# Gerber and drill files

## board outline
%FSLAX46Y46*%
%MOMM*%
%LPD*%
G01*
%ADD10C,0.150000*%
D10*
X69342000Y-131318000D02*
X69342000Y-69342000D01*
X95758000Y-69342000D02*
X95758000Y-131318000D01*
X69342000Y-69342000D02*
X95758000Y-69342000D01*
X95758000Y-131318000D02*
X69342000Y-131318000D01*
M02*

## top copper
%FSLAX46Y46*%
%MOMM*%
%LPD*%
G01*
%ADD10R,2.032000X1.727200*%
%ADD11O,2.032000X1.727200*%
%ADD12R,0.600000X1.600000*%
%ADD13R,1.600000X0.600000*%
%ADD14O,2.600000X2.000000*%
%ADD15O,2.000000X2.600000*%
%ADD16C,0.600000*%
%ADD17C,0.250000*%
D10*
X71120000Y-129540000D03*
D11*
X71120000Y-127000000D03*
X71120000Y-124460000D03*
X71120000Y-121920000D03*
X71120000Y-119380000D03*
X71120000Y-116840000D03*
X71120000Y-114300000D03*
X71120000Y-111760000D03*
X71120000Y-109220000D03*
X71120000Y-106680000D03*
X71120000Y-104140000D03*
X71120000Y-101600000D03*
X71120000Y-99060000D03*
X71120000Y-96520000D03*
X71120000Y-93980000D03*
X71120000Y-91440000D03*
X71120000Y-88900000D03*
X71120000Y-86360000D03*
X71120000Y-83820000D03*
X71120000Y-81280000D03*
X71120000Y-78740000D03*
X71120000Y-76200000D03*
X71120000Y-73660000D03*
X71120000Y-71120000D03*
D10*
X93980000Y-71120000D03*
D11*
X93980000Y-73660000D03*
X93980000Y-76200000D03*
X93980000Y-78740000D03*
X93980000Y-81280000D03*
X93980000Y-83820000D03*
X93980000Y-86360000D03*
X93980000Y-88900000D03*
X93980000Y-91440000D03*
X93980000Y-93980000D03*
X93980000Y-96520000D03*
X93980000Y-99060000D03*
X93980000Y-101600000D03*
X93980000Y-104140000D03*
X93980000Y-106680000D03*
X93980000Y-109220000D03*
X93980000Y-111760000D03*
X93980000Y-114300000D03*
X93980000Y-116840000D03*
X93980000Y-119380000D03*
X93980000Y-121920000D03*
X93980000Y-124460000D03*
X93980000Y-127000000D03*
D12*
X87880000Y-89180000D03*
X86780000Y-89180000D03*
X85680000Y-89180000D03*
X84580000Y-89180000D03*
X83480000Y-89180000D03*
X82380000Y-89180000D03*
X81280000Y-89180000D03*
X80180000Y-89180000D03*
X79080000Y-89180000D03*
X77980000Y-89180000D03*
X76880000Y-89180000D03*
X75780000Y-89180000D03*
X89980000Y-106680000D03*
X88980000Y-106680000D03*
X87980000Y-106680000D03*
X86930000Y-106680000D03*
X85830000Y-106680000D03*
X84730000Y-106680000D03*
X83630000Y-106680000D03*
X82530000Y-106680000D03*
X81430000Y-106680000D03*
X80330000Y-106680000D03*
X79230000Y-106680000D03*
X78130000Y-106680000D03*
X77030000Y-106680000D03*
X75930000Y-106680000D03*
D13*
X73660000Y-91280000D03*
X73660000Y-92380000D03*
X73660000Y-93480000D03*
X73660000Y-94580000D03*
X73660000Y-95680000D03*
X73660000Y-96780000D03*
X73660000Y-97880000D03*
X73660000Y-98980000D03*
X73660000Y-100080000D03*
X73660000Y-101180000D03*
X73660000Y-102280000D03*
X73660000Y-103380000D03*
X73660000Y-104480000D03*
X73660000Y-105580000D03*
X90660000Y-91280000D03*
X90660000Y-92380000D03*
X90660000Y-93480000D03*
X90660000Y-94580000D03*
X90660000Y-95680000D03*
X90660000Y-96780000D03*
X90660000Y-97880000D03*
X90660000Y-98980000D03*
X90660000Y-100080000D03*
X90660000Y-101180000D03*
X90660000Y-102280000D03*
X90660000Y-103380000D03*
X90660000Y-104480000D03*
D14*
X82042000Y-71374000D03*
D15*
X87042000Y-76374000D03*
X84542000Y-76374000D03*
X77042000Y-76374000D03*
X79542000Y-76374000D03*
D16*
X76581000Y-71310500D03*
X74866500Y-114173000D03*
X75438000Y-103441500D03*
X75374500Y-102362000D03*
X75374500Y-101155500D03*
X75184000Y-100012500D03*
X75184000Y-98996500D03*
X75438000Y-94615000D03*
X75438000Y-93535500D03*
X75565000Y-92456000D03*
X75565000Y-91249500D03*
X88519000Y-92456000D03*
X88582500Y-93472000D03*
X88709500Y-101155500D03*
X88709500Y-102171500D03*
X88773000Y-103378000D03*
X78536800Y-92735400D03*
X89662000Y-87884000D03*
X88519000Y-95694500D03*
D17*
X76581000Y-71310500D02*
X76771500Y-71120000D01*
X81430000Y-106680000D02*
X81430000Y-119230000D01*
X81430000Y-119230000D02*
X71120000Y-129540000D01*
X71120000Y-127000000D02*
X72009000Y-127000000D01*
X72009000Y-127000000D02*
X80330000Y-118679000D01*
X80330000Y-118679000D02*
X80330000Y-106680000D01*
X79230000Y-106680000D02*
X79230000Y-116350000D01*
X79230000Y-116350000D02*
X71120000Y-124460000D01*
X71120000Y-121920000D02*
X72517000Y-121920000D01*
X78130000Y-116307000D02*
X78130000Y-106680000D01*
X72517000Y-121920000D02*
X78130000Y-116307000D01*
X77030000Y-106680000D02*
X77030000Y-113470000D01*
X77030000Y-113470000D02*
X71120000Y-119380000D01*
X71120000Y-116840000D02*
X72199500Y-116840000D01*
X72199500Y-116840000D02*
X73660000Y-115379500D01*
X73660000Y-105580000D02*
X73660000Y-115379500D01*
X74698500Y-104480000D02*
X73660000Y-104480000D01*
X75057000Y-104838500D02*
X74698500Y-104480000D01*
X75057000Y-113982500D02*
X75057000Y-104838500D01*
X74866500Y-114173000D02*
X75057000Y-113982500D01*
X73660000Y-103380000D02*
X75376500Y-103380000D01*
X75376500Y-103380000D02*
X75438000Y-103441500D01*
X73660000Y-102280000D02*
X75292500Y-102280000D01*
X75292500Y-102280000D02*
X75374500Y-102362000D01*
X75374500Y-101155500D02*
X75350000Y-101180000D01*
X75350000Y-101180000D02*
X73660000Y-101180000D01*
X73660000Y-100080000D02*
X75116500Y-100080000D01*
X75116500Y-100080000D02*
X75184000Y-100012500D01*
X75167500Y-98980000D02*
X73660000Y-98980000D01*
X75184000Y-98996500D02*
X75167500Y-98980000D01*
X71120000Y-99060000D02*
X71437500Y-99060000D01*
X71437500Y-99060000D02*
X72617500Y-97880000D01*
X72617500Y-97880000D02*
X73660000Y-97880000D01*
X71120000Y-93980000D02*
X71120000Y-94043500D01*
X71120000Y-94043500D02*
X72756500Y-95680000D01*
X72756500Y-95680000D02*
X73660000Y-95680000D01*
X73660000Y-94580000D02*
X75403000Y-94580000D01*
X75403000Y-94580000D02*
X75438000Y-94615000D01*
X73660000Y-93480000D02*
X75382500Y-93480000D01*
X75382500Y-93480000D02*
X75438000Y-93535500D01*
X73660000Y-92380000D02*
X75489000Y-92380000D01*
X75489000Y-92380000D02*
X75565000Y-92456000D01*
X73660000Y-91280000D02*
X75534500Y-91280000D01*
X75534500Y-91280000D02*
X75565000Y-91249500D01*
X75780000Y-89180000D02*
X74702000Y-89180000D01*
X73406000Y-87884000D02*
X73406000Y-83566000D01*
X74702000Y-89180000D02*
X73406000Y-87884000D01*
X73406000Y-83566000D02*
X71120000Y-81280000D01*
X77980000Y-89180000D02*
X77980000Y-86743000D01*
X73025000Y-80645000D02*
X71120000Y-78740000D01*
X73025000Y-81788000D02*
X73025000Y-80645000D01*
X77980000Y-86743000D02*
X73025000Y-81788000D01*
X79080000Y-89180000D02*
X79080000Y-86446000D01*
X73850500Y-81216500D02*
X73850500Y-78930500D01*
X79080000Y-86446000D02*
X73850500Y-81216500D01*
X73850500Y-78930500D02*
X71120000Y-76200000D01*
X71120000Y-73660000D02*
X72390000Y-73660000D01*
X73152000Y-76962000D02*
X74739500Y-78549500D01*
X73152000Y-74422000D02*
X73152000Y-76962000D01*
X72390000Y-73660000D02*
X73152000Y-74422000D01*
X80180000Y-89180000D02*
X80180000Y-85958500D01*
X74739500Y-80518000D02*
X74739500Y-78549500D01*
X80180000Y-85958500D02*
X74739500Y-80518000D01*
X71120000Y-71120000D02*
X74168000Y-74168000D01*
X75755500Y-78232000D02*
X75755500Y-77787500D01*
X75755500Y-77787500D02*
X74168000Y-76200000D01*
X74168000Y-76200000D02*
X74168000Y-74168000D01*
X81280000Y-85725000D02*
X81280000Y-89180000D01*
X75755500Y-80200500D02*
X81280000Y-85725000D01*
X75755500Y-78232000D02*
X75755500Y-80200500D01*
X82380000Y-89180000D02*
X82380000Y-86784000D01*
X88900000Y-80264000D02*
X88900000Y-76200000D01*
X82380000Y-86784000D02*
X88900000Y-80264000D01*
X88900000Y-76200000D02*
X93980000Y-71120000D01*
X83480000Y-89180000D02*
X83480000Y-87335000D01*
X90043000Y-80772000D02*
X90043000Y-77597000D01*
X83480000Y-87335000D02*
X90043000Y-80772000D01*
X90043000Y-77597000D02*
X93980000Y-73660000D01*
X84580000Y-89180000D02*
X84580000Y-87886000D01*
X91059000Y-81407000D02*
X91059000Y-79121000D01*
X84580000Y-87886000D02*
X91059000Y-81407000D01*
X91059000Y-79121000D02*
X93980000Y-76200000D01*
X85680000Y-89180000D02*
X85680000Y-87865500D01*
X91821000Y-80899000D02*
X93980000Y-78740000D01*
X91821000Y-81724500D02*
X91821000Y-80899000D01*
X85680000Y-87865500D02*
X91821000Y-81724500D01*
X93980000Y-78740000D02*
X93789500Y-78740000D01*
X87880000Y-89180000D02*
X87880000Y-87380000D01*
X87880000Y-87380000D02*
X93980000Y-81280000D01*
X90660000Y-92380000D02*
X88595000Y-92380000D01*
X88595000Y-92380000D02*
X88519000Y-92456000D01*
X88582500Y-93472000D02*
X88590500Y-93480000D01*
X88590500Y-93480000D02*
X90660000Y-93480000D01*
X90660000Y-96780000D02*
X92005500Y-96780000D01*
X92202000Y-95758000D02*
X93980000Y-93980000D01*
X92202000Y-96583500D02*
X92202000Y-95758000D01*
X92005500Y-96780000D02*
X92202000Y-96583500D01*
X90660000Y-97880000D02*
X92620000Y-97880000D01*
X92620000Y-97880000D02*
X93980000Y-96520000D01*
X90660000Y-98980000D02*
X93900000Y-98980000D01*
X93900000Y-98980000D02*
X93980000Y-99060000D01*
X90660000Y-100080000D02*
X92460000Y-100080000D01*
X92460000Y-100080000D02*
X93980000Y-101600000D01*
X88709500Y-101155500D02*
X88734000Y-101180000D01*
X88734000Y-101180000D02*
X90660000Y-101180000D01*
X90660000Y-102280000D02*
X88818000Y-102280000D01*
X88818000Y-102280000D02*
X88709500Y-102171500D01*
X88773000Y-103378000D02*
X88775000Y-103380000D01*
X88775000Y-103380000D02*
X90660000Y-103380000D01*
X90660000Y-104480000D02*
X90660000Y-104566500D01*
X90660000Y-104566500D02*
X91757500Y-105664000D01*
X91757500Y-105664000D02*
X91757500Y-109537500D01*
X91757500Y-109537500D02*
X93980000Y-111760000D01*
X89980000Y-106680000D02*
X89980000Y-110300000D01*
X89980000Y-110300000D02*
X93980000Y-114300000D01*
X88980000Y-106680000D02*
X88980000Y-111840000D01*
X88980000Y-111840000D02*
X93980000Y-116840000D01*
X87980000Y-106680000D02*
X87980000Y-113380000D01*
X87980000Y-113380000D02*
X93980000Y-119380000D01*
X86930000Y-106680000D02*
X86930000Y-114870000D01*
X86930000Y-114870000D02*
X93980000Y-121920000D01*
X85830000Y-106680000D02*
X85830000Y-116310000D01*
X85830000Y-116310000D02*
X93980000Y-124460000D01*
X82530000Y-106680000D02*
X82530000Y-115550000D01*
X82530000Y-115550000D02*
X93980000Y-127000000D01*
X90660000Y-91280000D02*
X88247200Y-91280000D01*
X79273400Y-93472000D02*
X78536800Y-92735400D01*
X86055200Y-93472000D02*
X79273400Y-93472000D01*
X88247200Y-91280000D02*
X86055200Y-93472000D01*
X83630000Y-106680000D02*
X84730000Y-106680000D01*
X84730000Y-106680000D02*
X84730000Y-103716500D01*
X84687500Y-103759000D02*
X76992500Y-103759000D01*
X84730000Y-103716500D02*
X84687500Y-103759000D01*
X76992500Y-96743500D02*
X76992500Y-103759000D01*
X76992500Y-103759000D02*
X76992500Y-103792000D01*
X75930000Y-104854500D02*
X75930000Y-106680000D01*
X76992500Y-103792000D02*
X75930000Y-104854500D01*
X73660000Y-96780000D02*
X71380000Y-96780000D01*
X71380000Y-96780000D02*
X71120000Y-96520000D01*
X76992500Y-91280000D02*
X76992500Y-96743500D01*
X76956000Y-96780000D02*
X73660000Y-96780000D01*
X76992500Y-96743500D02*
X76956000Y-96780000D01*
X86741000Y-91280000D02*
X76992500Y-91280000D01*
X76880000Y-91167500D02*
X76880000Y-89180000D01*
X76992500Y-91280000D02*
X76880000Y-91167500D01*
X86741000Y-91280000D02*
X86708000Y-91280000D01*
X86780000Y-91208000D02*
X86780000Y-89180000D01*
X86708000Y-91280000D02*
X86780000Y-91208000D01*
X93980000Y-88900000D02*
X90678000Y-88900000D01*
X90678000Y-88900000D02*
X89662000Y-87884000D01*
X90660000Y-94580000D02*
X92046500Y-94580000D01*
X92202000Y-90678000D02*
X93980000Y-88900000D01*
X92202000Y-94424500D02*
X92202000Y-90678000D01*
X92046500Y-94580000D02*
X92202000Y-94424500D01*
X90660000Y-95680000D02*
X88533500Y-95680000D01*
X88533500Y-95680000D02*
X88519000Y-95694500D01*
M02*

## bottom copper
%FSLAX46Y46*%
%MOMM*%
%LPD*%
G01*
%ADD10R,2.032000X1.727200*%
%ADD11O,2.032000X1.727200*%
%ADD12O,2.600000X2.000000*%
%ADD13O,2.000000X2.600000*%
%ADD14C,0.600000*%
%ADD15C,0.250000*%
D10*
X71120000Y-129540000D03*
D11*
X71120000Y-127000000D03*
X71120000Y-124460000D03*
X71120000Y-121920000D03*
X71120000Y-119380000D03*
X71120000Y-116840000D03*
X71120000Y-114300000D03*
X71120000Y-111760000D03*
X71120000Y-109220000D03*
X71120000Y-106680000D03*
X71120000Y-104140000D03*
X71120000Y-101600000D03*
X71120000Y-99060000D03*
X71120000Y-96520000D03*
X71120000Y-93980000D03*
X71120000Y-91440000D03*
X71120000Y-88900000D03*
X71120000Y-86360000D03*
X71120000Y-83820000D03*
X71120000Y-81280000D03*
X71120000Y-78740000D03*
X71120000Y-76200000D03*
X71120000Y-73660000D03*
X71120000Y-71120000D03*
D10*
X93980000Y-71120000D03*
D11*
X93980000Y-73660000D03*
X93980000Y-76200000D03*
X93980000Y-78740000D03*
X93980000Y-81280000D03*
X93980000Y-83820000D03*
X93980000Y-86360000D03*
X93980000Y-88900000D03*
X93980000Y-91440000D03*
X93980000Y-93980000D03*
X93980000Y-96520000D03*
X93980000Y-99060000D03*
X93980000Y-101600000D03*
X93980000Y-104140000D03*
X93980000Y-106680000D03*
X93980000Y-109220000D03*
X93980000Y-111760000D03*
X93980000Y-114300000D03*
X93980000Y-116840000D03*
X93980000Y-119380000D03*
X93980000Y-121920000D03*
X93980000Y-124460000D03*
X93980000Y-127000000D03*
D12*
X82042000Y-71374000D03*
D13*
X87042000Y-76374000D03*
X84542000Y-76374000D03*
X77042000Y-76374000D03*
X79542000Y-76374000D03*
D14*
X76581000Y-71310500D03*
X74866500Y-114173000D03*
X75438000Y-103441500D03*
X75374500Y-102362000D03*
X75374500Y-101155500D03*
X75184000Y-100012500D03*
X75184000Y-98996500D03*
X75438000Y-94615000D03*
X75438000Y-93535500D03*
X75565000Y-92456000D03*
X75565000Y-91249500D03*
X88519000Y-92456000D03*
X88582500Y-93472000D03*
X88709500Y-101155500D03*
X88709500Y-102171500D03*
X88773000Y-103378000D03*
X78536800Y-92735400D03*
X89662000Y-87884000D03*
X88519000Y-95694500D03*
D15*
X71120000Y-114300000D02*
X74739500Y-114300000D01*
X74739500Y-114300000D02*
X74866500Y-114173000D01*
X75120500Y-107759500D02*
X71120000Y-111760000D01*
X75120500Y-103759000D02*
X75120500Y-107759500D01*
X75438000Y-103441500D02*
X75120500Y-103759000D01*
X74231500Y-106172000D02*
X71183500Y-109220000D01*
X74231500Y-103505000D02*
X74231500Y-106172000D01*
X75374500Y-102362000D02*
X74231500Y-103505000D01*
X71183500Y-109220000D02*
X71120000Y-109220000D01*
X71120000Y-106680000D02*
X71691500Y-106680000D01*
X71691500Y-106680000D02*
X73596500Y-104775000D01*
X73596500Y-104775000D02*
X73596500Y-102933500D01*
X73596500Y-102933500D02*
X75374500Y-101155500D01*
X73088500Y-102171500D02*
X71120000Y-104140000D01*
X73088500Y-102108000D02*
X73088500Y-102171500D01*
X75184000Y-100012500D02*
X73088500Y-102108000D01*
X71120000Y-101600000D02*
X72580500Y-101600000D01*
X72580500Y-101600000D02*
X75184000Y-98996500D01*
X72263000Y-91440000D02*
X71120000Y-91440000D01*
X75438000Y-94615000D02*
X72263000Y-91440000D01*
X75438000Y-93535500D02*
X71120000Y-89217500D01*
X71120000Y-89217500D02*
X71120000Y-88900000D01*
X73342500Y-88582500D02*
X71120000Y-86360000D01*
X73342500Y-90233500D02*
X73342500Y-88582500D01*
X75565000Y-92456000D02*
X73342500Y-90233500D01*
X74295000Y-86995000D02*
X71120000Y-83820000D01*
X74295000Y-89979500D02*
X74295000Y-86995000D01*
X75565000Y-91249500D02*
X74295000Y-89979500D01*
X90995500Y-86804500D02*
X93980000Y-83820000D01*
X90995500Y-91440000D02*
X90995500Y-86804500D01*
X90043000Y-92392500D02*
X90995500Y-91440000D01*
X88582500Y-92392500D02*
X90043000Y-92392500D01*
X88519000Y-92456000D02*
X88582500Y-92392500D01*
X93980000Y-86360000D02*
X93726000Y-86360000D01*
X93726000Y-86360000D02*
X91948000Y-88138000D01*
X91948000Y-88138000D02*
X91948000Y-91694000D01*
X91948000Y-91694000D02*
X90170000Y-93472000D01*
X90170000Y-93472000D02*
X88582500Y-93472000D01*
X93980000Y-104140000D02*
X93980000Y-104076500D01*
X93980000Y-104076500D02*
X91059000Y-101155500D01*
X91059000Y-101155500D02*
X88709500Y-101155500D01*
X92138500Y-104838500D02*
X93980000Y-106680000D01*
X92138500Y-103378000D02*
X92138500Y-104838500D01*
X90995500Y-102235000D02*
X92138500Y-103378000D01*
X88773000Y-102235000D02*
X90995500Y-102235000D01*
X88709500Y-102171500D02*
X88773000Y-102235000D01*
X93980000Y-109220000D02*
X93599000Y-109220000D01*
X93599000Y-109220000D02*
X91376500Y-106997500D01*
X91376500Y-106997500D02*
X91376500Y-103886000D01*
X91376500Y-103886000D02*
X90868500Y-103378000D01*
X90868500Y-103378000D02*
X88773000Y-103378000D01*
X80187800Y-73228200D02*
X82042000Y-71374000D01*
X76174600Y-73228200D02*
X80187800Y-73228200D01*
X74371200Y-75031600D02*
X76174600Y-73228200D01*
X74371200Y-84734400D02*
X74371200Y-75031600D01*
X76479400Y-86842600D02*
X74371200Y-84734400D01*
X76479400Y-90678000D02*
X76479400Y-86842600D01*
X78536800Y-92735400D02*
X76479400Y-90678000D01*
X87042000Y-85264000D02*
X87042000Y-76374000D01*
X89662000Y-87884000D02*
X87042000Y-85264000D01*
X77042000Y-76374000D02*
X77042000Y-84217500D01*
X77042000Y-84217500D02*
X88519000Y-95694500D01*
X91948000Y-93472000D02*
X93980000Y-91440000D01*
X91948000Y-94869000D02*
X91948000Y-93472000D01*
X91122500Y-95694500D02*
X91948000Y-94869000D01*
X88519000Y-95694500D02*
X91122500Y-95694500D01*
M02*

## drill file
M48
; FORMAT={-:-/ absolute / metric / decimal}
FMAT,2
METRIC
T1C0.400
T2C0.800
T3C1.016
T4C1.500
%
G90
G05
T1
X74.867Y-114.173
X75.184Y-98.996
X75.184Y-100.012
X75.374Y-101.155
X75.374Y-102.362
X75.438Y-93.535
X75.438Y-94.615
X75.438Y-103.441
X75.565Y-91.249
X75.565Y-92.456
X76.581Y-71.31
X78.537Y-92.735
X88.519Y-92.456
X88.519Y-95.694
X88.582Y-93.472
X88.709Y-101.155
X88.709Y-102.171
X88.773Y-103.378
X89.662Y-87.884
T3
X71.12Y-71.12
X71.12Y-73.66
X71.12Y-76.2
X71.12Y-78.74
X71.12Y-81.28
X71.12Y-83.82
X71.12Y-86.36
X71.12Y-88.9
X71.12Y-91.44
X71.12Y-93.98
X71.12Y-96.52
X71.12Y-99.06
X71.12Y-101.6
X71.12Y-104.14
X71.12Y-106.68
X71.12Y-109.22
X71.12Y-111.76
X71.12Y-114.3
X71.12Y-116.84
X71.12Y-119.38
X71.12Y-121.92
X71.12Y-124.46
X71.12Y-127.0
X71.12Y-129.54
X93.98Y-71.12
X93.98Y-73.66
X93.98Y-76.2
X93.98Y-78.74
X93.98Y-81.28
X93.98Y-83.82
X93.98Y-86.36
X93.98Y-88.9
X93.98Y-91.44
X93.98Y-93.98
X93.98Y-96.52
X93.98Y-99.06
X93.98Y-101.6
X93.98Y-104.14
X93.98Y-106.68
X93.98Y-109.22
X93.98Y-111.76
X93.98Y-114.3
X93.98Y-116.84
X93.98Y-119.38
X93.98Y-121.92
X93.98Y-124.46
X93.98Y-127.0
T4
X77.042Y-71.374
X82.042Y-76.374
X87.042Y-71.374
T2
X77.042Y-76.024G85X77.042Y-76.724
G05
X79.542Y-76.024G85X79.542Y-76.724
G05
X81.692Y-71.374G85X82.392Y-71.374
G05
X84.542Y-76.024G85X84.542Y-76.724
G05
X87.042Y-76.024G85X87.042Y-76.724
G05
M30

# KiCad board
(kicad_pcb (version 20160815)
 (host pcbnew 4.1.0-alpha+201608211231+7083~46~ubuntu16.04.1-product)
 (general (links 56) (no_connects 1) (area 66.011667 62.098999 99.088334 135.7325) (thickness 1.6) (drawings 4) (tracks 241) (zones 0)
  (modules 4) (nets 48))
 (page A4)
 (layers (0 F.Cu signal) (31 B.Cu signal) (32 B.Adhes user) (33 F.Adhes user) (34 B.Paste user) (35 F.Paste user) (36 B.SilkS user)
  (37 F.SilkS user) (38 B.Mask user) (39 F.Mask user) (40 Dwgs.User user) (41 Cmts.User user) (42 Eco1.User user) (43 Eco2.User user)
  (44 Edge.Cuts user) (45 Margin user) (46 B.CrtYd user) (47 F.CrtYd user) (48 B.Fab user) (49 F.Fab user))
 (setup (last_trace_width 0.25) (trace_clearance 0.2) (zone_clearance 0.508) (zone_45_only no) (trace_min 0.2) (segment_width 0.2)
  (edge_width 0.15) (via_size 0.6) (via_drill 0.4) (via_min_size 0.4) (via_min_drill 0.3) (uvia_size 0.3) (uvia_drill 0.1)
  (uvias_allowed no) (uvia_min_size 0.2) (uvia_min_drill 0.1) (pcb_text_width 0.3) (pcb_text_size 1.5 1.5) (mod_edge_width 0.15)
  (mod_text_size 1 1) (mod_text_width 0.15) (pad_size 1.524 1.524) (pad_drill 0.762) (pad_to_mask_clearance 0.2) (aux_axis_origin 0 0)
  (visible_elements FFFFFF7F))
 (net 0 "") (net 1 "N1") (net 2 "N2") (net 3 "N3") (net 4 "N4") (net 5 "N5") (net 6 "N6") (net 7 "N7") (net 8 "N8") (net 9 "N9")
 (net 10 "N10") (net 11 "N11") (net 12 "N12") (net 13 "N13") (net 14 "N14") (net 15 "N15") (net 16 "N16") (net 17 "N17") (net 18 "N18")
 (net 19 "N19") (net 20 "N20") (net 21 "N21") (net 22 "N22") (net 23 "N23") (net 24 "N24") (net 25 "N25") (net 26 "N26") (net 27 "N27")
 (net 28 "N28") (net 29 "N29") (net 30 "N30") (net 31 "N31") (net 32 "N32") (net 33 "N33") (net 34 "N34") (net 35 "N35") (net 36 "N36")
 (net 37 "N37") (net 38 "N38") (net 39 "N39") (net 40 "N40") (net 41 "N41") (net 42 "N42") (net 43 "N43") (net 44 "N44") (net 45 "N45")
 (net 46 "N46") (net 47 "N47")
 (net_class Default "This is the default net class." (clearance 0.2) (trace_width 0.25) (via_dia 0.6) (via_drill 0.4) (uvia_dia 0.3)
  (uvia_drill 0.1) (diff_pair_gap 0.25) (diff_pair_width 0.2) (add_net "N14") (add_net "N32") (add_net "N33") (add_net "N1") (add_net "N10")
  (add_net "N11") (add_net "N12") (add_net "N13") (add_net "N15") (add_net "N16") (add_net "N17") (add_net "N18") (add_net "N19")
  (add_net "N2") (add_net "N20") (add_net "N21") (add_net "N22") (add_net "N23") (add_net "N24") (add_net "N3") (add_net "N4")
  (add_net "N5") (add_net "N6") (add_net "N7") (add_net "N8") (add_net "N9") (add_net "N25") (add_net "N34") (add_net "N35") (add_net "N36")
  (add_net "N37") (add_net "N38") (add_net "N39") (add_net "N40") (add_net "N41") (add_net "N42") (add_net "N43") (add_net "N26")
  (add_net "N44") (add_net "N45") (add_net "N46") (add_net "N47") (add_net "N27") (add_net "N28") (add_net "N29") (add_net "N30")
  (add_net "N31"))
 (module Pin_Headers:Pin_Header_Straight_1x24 (layer F.Cu) (at 71.12 129.54 180)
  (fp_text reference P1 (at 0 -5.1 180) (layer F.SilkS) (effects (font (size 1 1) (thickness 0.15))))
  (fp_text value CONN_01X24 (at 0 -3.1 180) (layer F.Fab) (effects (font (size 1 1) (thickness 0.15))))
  (pad 1 thru_hole rect (at 0 0 180) (size 2.032 1.7272) (drill 1.016) (layers *.Cu *.Mask F.SilkS) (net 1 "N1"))
  (pad 2 thru_hole oval (at 0 2.54 180) (size 2.032 1.7272) (drill 1.016) (layers *.Cu *.Mask F.SilkS) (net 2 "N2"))
  (pad 3 thru_hole oval (at 0 5.08 180) (size 2.032 1.7272) (drill 1.016) (layers *.Cu *.Mask F.SilkS) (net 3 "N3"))
  (pad 4 thru_hole oval (at 0 7.62 180) (size 2.032 1.7272) (drill 1.016) (layers *.Cu *.Mask F.SilkS) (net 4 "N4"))
  (pad 5 thru_hole oval (at 0 10.16 180) (size 2.032 1.7272) (drill 1.016) (layers *.Cu *.Mask F.SilkS) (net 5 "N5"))
  (pad 6 thru_hole oval (at 0 12.7 180) (size 2.032 1.7272) (drill 1.016) (layers *.Cu *.Mask F.SilkS) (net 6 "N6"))
  (pad 7 thru_hole oval (at 0 15.24 180) (size 2.032 1.7272) (drill 1.016) (layers *.Cu *.Mask F.SilkS) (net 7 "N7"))
  (pad 8 thru_hole oval (at 0 17.78 180) (size 2.032 1.7272) (drill 1.016) (layers *.Cu *.Mask F.SilkS) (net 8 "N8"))
  (pad 9 thru_hole oval (at 0 20.32 180) (size 2.032 1.7272) (drill 1.016) (layers *.Cu *.Mask F.SilkS) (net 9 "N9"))
  (pad 10 thru_hole oval (at 0 22.86 180) (size 2.032 1.7272) (drill 1.016) (layers *.Cu *.Mask F.SilkS) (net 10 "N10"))
  (pad 11 thru_hole oval (at 0 25.4 180) (size 2.032 1.7272) (drill 1.016) (layers *.Cu *.Mask F.SilkS) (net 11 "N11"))
  (pad 12 thru_hole oval (at 0 27.94 180) (size 2.032 1.7272) (drill 1.016) (layers *.Cu *.Mask F.SilkS) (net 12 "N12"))
  (pad 13 thru_hole oval (at 0 30.48 180) (size 2.032 1.7272) (drill 1.016) (layers *.Cu *.Mask F.SilkS) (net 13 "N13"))
  (pad 14 thru_hole oval (at 0 33.02 180) (size 2.032 1.7272) (drill 1.016) (layers *.Cu *.Mask F.SilkS) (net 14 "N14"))
  (pad 15 thru_hole oval (at 0 35.56 180) (size 2.032 1.7272) (drill 1.016) (layers *.Cu *.Mask F.SilkS) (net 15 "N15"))
  (pad 16 thru_hole oval (at 0 38.1 180) (size 2.032 1.7272) (drill 1.016) (layers *.Cu *.Mask F.SilkS) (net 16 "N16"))
  (pad 17 thru_hole oval (at 0 40.64 180) (size 2.032 1.7272) (drill 1.016) (layers *.Cu *.Mask F.SilkS) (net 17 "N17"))
  (pad 18 thru_hole oval (at 0 43.18 180) (size 2.032 1.7272) (drill 1.016) (layers *.Cu *.Mask F.SilkS) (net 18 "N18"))
  (pad 19 thru_hole oval (at 0 45.72 180) (size 2.032 1.7272) (drill 1.016) (layers *.Cu *.Mask F.SilkS) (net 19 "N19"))
  (pad 20 thru_hole oval (at 0 48.26 180) (size 2.032 1.7272) (drill 1.016) (layers *.Cu *.Mask F.SilkS) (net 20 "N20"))
  (pad 21 thru_hole oval (at 0 50.8 180) (size 2.032 1.7272) (drill 1.016) (layers *.Cu *.Mask F.SilkS) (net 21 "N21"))
  (pad 22 thru_hole oval (at 0 53.34 180) (size 2.032 1.7272) (drill 1.016) (layers *.Cu *.Mask F.SilkS) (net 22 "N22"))
  (pad 23 thru_hole oval (at 0 55.88 180) (size 2.032 1.7272) (drill 1.016) (layers *.Cu *.Mask F.SilkS) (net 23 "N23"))
  (pad 24 thru_hole oval (at 0 58.42 180) (size 2.032 1.7272) (drill 1.016) (layers *.Cu *.Mask F.SilkS) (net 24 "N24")))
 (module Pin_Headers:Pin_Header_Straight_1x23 (layer F.Cu) (at 93.98 71.12)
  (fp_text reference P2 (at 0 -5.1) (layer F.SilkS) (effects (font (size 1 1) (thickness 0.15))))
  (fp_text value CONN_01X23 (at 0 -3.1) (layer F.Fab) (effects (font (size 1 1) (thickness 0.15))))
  (pad 1 thru_hole rect (at 0 0) (size 2.032 1.7272) (drill 1.016) (layers *.Cu *.Mask F.SilkS) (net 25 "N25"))
  (pad 2 thru_hole oval (at 0 2.54) (size 2.032 1.7272) (drill 1.016) (layers *.Cu *.Mask F.SilkS) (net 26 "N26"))
  (pad 3 thru_hole oval (at 0 5.08) (size 2.032 1.7272) (drill 1.016) (layers *.Cu *.Mask F.SilkS) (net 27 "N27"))
  (pad 4 thru_hole oval (at 0 7.62) (size 2.032 1.7272) (drill 1.016) (layers *.Cu *.Mask F.SilkS) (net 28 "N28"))
  (pad 5 thru_hole oval (at 0 10.16) (size 2.032 1.7272) (drill 1.016) (layers *.Cu *.Mask F.SilkS) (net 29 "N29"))
  (pad 6 thru_hole oval (at 0 12.7) (size 2.032 1.7272) (drill 1.016) (layers *.Cu *.Mask F.SilkS) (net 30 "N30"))
  (pad 7 thru_hole oval (at 0 15.24) (size 2.032 1.7272) (drill 1.016) (layers *.Cu *.Mask F.SilkS) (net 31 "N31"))
  (pad 8 thru_hole oval (at 0 17.78) (size 2.032 1.7272) (drill 1.016) (layers *.Cu *.Mask F.SilkS) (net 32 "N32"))
  (pad 9 thru_hole oval (at 0 20.32) (size 2.032 1.7272) (drill 1.016) (layers *.Cu *.Mask F.SilkS) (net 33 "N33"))
  (pad 10 thru_hole oval (at 0 22.86) (size 2.032 1.7272) (drill 1.016) (layers *.Cu *.Mask F.SilkS) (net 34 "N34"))
  (pad 11 thru_hole oval (at 0 25.4) (size 2.032 1.7272) (drill 1.016) (layers *.Cu *.Mask F.SilkS) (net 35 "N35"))
  (pad 12 thru_hole oval (at 0 27.94) (size 2.032 1.7272) (drill 1.016) (layers *.Cu *.Mask F.SilkS) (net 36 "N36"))
  (pad 13 thru_hole oval (at 0 30.48) (size 2.032 1.7272) (drill 1.016) (layers *.Cu *.Mask F.SilkS) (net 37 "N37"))
  (pad 14 thru_hole oval (at 0 33.02) (size 2.032 1.7272) (drill 1.016) (layers *.Cu *.Mask F.SilkS) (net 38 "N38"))
  (pad 15 thru_hole oval (at 0 35.56) (size 2.032 1.7272) (drill 1.016) (layers *.Cu *.Mask F.SilkS) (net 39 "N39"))
  (pad 16 thru_hole oval (at 0 38.1) (size 2.032 1.7272) (drill 1.016) (layers *.Cu *.Mask F.SilkS) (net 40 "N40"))
  (pad 17 thru_hole oval (at 0 40.64) (size 2.032 1.7272) (drill 1.016) (layers *.Cu *.Mask F.SilkS) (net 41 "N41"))
  (pad 18 thru_hole oval (at 0 43.18) (size 2.032 1.7272) (drill 1.016) (layers *.Cu *.Mask F.SilkS) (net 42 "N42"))
  (pad 19 thru_hole oval (at 0 45.72) (size 2.032 1.7272) (drill 1.016) (layers *.Cu *.Mask F.SilkS) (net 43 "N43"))
  (pad 20 thru_hole oval (at 0 48.26) (size 2.032 1.7272) (drill 1.016) (layers *.Cu *.Mask F.SilkS) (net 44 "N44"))
  (pad 21 thru_hole oval (at 0 50.8) (size 2.032 1.7272) (drill 1.016) (layers *.Cu *.Mask F.SilkS) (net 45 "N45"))
  (pad 22 thru_hole oval (at 0 53.34) (size 2.032 1.7272) (drill 1.016) (layers *.Cu *.Mask F.SilkS) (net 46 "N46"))
  (pad 23 thru_hole oval (at 0 55.88) (size 2.032 1.7272) (drill 1.016) (layers *.Cu *.Mask F.SilkS) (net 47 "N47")))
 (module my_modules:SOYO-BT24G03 (layer F.Cu) (at 73.66 106.68)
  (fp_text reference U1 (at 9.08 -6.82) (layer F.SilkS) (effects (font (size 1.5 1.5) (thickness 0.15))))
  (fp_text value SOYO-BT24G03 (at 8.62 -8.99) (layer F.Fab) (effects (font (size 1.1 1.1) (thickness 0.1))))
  (pad 39 smd rect (at 14.22 -17.5) (size 0.6 1.6) (layers F.Cu F.Paste F.Mask) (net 29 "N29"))
  (pad 40 smd rect (at 13.12 -17.5) (size 0.6 1.6) (layers F.Cu F.Paste F.Mask) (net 14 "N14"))
  (pad 41 smd rect (at 12.02 -17.5) (size 0.6 1.6) (layers F.Cu F.Paste F.Mask) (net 28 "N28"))
  (pad 42 smd rect (at 10.92 -17.5) (size 0.6 1.6) (layers F.Cu F.Paste F.Mask) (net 27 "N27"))
  (pad 43 smd rect (at 9.82 -17.5) (size 0.6 1.6) (layers F.Cu F.Paste F.Mask) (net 26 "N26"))
  (pad 44 smd rect (at 8.72 -17.5) (size 0.6 1.6) (layers F.Cu F.Paste F.Mask) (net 25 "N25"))
  (pad 45 smd rect (at 7.62 -17.5) (size 0.6 1.6) (layers F.Cu F.Paste F.Mask) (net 24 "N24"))
  (pad 46 smd rect (at 6.52 -17.5) (size 0.6 1.6) (layers F.Cu F.Paste F.Mask) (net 23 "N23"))
  (pad 47 smd rect (at 5.42 -17.5) (size 0.6 1.6) (layers F.Cu F.Paste F.Mask) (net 22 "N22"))
  (pad 48 smd rect (at 4.32 -17.5) (size 0.6 1.6) (layers F.Cu F.Paste F.Mask) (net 21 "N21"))
  (pad 49 smd rect (at 3.22 -17.5) (size 0.6 1.6) (layers F.Cu F.Paste F.Mask) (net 14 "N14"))
  (pad 50 smd rect (at 2.12 -17.5) (size 0.6 1.6) (layers F.Cu F.Paste F.Mask) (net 20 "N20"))
  (pad 52 smd rect (at 16.32 0) (size 0.6 1.6) (layers F.Cu F.Paste F.Mask) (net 42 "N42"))
  (pad 51 smd rect (at 15.32 0) (size 0.6 1.6) (layers F.Cu F.Paste F.Mask) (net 43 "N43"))
  (pad 25 smd rect (at 14.32 0) (size 0.6 1.6) (layers F.Cu F.Paste F.Mask) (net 44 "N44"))
  (pad 24 smd rect (at 13.27 0) (size 0.6 1.6) (layers F.Cu F.Paste F.Mask) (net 45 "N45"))
  (pad 23 smd rect (at 12.17 0) (size 0.6 1.6) (layers F.Cu F.Paste F.Mask) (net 46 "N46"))
  (pad 22 smd rect (at 11.07 0) (size 0.6 1.6) (layers F.Cu F.Paste F.Mask) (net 14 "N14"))
  (pad 21 smd rect (at 9.97 0) (size 0.6 1.6) (layers F.Cu F.Paste F.Mask) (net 14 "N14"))
  (pad 20 smd rect (at 8.87 0) (size 0.6 1.6) (layers F.Cu F.Paste F.Mask) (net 47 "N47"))
  (pad 19 smd rect (at 7.77 0) (size 0.6 1.6) (layers F.Cu F.Paste F.Mask) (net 1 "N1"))
  (pad 18 smd rect (at 6.67 0) (size 0.6 1.6) (layers F.Cu F.Paste F.Mask) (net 2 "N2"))
  (pad 17 smd rect (at 5.57 0) (size 0.6 1.6) (layers F.Cu F.Paste F.Mask) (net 3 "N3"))
  (pad 16 smd rect (at 4.47 0) (size 0.6 1.6) (layers F.Cu F.Paste F.Mask) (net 4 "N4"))
  (pad 15 smd rect (at 3.37 0) (size 0.6 1.6) (layers F.Cu F.Paste F.Mask) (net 5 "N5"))
  (pad 14 smd rect (at 2.27 0) (size 0.6 1.6) (layers F.Cu F.Paste F.Mask) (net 14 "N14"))
  (pad 1 smd rect (at 0 -15.4) (size 1.6 0.6) (layers F.Cu F.Paste F.Mask) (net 19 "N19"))
  (pad 2 smd rect (at 0 -14.3) (size 1.6 0.6) (layers F.Cu F.Paste F.Mask) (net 18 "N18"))
  (pad 3 smd rect (at 0 -13.2) (size 1.6 0.6) (layers F.Cu F.Paste F.Mask) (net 17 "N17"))
  (pad 4 smd rect (at 0 -12.1) (size 1.6 0.6) (layers F.Cu F.Paste F.Mask) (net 16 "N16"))
  (pad 5 smd rect (at 0 -11) (size 1.6 0.6) (layers F.Cu F.Paste F.Mask) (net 15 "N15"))
  (pad 6 smd rect (at 0 -9.9) (size 1.6 0.6) (layers F.Cu F.Paste F.Mask) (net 14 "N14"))
  (pad 7 smd rect (at 0 -8.8) (size 1.6 0.6) (layers F.Cu F.Paste F.Mask) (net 13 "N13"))
  (pad 8 smd rect (at 0 -7.7) (size 1.6 0.6) (layers F.Cu F.Paste F.Mask) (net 12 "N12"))
  (pad 9 smd rect (at 0 -6.6) (size 1.6 0.6) (layers F.Cu F.Paste F.Mask) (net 11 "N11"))
  (pad 10 smd rect (at 0 -5.5) (size 1.6 0.6) (layers F.Cu F.Paste F.Mask) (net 10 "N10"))
  (pad 11 smd rect (at 0 -4.4) (size 1.6 0.6) (layers F.Cu F.Paste F.Mask) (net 9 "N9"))
  (pad 12 smd rect (at 0 -3.3) (size 1.6 0.6) (layers F.Cu F.Paste F.Mask) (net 8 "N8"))
  (pad 13 smd rect (at 0 -2.2) (size 1.6 0.6) (layers F.Cu F.Paste F.Mask) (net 7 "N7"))
  (pad 53 smd rect (at 0 -1.1) (size 1.6 0.6) (layers F.Cu F.Paste F.Mask) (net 6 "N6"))
  (pad 38 smd rect (at 17 -15.4) (size 1.6 0.6) (layers F.Cu F.Paste F.Mask) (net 14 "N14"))
  (pad 37 smd rect (at 17 -14.3) (size 1.6 0.6) (layers F.Cu F.Paste F.Mask) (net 30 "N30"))
  (pad 36 smd rect (at 17 -13.2) (size 1.6 0.6) (layers F.Cu F.Paste F.Mask) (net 31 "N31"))
  (pad 35 smd rect (at 17 -12.1) (size 1.6 0.6) (layers F.Cu F.Paste F.Mask) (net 32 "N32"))
  (pad 34 smd rect (at 17 -11) (size 1.6 0.6) (layers F.Cu F.Paste F.Mask) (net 33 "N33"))
  (pad 33 smd rect (at 17 -9.9) (size 1.6 0.6) (layers F.Cu F.Paste F.Mask) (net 34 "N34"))
  (pad 32 smd rect (at 17 -8.8) (size 1.6 0.6) (layers F.Cu F.Paste F.Mask) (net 35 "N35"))
  (pad 31 smd rect (at 17 -7.7) (size 1.6 0.6) (layers F.Cu F.Paste F.Mask) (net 36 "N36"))
  (pad 30 smd rect (at 17 -6.6) (size 1.6 0.6) (layers F.Cu F.Paste F.Mask) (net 37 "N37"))
  (pad 29 smd rect (at 17 -5.5) (size 1.6 0.6) (layers F.Cu F.Paste F.Mask) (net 38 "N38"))
  (pad 28 smd rect (at 17 -4.4) (size 1.6 0.6) (layers F.Cu F.Paste F.Mask) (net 39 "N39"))
  (pad 27 smd rect (at 17 -3.3) (size 1.6 0.6) (layers F.Cu F.Paste F.Mask) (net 40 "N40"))
  (pad 26 smd rect (at 17 -2.2) (size 1.6 0.6) (layers F.Cu F.Paste F.Mask) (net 41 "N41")))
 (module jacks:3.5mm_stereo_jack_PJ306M (layer F.Cu) (at 82.042 71.374)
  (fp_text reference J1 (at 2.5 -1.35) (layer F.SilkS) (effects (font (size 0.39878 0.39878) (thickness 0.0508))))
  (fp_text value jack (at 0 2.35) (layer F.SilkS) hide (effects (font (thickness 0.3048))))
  (pad 1 thru_hole oval (at 0 0) (size 2.6 2) (drill oval 1.5 0.8) (layers *.Cu *.Mask F.SilkS) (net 14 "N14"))
  (pad 2 thru_hole oval (at 5 5) (size 2 2.6) (drill oval 0.8 1.5) (layers *.Cu *.Mask F.SilkS) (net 32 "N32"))
  (pad 3 thru_hole oval (at 2.5 5) (size 2 2.6) (drill oval 0.8 1.5) (layers *.Cu *.Mask F.SilkS))
  (pad 5 thru_hole oval (at -5 5) (size 2 2.6) (drill oval 0.8 1.5) (layers *.Cu *.Mask F.SilkS) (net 33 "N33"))
  (pad 4 thru_hole oval (at -2.5 5) (size 2 2.6) (drill oval 0.8 1.5) (layers *.Cu *.Mask F.SilkS))
  (pad "" np_thru_hole circle (at 0 5) (size 1.5 1.5) (drill 1.5) (layers *.Cu *.Mask F.SilkS))
  (pad "" np_thru_hole circle (at 5 0) (size 1.5 1.5) (drill 1.5) (layers *.Cu *.Mask F.SilkS))
  (pad "" np_thru_hole circle (at -5 0) (size 1.5 1.5) (drill 1.5) (layers *.Cu *.Mask F.SilkS)))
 (gr_line (start 69.342 131.318) (end 69.342 69.342) (angle 90) (layer Edge.Cuts) (width 0.15))
 (gr_line (start 95.758 69.342) (end 95.758 131.318) (angle 90) (layer Edge.Cuts) (width 0.15))
 (gr_line (start 69.342 69.342) (end 95.758 69.342) (angle 90) (layer Edge.Cuts) (width 0.15))
 (gr_line (start 95.758 131.318) (end 69.342 131.318) (angle 90) (layer Edge.Cuts) (width 0.15))
 (segment (start 76.581 71.3105) (end 76.7715 71.12) (width 0.25) (layer F.Cu) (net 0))
 (via (at 76.581 71.3105) (size 0.6) (drill 0.4) (layers F.Cu B.Cu) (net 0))
 (segment (start 81.43 106.68) (end 81.43 119.23) (width 0.25) (layer F.Cu) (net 1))
 (segment (start 81.43 119.23) (end 71.12 129.54) (width 0.25) (layer F.Cu) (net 1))
 (segment (start 71.12 127) (end 72.009 127) (width 0.25) (layer F.Cu) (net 2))
 (segment (start 72.009 127) (end 80.33 118.679) (width 0.25) (layer F.Cu) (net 2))
 (segment (start 80.33 118.679) (end 80.33 106.68) (width 0.25) (layer F.Cu) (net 2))
 (segment (start 79.23 106.68) (end 79.23 116.35) (width 0.25) (layer F.Cu) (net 3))
 (segment (start 79.23 116.35) (end 71.12 124.46) (width 0.25) (layer F.Cu) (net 3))
 (segment (start 71.12 121.92) (end 72.517 121.92) (width 0.25) (layer F.Cu) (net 4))
 (segment (start 78.13 116.307) (end 78.13 106.68) (width 0.25) (layer F.Cu) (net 4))
 (segment (start 72.517 121.92) (end 78.13 116.307) (width 0.25) (layer F.Cu) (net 4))
 (segment (start 77.03 106.68) (end 77.03 113.47) (width 0.25) (layer F.Cu) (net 5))
 (segment (start 77.03 113.47) (end 71.12 119.38) (width 0.25) (layer F.Cu) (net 5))
 (segment (start 71.12 116.84) (end 72.1995 116.84) (width 0.25) (layer F.Cu) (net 6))
 (segment (start 72.1995 116.84) (end 73.66 115.3795) (width 0.25) (layer F.Cu) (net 6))
 (segment (start 73.66 105.58) (end 73.66 115.3795) (width 0.25) (layer F.Cu) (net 6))
 (segment (start 71.12 114.3) (end 74.7395 114.3) (width 0.25) (layer B.Cu) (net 7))
 (segment (start 74.6985 104.48) (end 73.66 104.48) (width 0.25) (layer F.Cu) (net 7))
 (segment (start 75.057 104.8385) (end 74.6985 104.48) (width 0.25) (layer F.Cu) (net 7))
 (segment (start 75.057 113.9825) (end 75.057 104.8385) (width 0.25) (layer F.Cu) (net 7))
 (segment (start 74.8665 114.173) (end 75.057 113.9825) (width 0.25) (layer F.Cu) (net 7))
 (via (at 74.8665 114.173) (size 0.6) (drill 0.4) (layers F.Cu B.Cu) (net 7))
 (segment (start 74.7395 114.3) (end 74.8665 114.173) (width 0.25) (layer B.Cu) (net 7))
 (segment (start 73.66 103.38) (end 75.3765 103.38) (width 0.25) (layer F.Cu) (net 8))
 (segment (start 75.1205 107.7595) (end 71.12 111.76) (width 0.25) (layer B.Cu) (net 8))
 (segment (start 75.1205 103.759) (end 75.1205 107.7595) (width 0.25) (layer B.Cu) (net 8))
 (segment (start 75.438 103.4415) (end 75.1205 103.759) (width 0.25) (layer B.Cu) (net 8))
 (via (at 75.438 103.4415) (size 0.6) (drill 0.4) (layers F.Cu B.Cu) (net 8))
 (segment (start 75.3765 103.38) (end 75.438 103.4415) (width 0.25) (layer F.Cu) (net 8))
 (segment (start 73.66 102.28) (end 75.2925 102.28) (width 0.25) (layer F.Cu) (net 9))
 (segment (start 74.2315 106.172) (end 71.1835 109.22) (width 0.25) (layer B.Cu) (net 9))
 (segment (start 74.2315 103.505) (end 74.2315 106.172) (width 0.25) (layer B.Cu) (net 9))
 (segment (start 75.3745 102.362) (end 74.2315 103.505) (width 0.25) (layer B.Cu) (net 9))
 (via (at 75.3745 102.362) (size 0.6) (drill 0.4) (layers F.Cu B.Cu) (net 9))
 (segment (start 75.2925 102.28) (end 75.3745 102.362) (width 0.25) (layer F.Cu) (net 9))
 (segment (start 71.1835 109.22) (end 71.12 109.22) (width 0.25) (layer B.Cu) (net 9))
 (segment (start 71.12 106.68) (end 71.6915 106.68) (width 0.25) (layer B.Cu) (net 10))
 (segment (start 71.6915 106.68) (end 73.5965 104.775) (width 0.25) (layer B.Cu) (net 10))
 (segment (start 73.5965 104.775) (end 73.5965 102.9335) (width 0.25) (layer B.Cu) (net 10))
 (segment (start 73.5965 102.9335) (end 75.3745 101.1555) (width 0.25) (layer B.Cu) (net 10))
 (via (at 75.3745 101.1555) (size 0.6) (drill 0.4) (layers F.Cu B.Cu) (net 10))
 (segment (start 75.3745 101.1555) (end 75.35 101.18) (width 0.25) (layer F.Cu) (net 10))
 (segment (start 75.35 101.18) (end 73.66 101.18) (width 0.25) (layer F.Cu) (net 10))
 (segment (start 73.66 100.08) (end 75.1165 100.08) (width 0.25) (layer F.Cu) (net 11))
 (segment (start 73.0885 102.1715) (end 71.12 104.14) (width 0.25) (layer B.Cu) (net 11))
 (segment (start 73.0885 102.108) (end 73.0885 102.1715) (width 0.25) (layer B.Cu) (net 11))
 (segment (start 75.184 100.0125) (end 73.0885 102.108) (width 0.25) (layer B.Cu) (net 11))
 (via (at 75.184 100.0125) (size 0.6) (drill 0.4) (layers F.Cu B.Cu) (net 11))
 (segment (start 75.1165 100.08) (end 75.184 100.0125) (width 0.25) (layer F.Cu) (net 11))
 (segment (start 71.12 101.6) (end 72.5805 101.6) (width 0.25) (layer B.Cu) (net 12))
 (segment (start 75.1675 98.98) (end 73.66 98.98) (width 0.25) (layer F.Cu) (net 12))
 (segment (start 75.184 98.9965) (end 75.1675 98.98) (width 0.25) (layer F.Cu) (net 12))
 (via (at 75.184 98.9965) (size 0.6) (drill 0.4) (layers F.Cu B.Cu) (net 12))
 (segment (start 72.5805 101.6) (end 75.184 98.9965) (width 0.25) (layer B.Cu) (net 12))
 (segment (start 71.12 99.06) (end 71.4375 99.06) (width 0.25) (layer F.Cu) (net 13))
 (segment (start 71.4375 99.06) (end 72.6175 97.88) (width 0.25) (layer F.Cu) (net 13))
 (segment (start 72.6175 97.88) (end 73.66 97.88) (width 0.25) (layer F.Cu) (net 13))
 (segment (start 71.12 93.98) (end 71.12 94.0435) (width 0.25) (layer F.Cu) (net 15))
 (segment (start 71.12 94.0435) (end 72.7565 95.68) (width 0.25) (layer F.Cu) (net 15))
 (segment (start 72.7565 95.68) (end 73.66 95.68) (width 0.25) (layer F.Cu) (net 15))
 (segment (start 73.66 94.58) (end 75.403 94.58) (width 0.25) (layer F.Cu) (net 16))
 (segment (start 72.263 91.44) (end 71.12 91.44) (width 0.25) (layer B.Cu) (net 16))
 (segment (start 75.438 94.615) (end 72.263 91.44) (width 0.25) (layer B.Cu) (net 16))
 (via (at 75.438 94.615) (size 0.6) (drill 0.4) (layers F.Cu B.Cu) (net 16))
 (segment (start 75.403 94.58) (end 75.438 94.615) (width 0.25) (layer F.Cu) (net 16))
 (segment (start 73.66 93.48) (end 75.3825 93.48) (width 0.25) (layer F.Cu) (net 17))
 (segment (start 75.438 93.5355) (end 71.12 89.2175) (width 0.25) (layer B.Cu) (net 17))
 (via (at 75.438 93.5355) (size 0.6) (drill 0.4) (layers F.Cu B.Cu) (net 17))
 (segment (start 75.3825 93.48) (end 75.438 93.5355) (width 0.25) (layer F.Cu) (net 17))
 (segment (start 71.12 89.2175) (end 71.12 88.9) (width 0.25) (layer B.Cu) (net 17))
 (segment (start 73.66 92.38) (end 75.489 92.38) (width 0.25) (layer F.Cu) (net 18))
 (segment (start 73.3425 88.5825) (end 71.12 86.36) (width 0.25) (layer B.Cu) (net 18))
 (segment (start 73.3425 90.2335) (end 73.3425 88.5825) (width 0.25) (layer B.Cu) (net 18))
 (segment (start 75.565 92.456) (end 73.3425 90.2335) (width 0.25) (layer B.Cu) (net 18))
 (via (at 75.565 92.456) (size 0.6) (drill 0.4) (layers F.Cu B.Cu) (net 18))
 (segment (start 75.489 92.38) (end 75.565 92.456) (width 0.25) (layer F.Cu) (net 18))
 (segment (start 73.66 91.28) (end 75.5345 91.28) (width 0.25) (layer F.Cu) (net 19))
 (segment (start 74.295 86.995) (end 71.12 83.82) (width 0.25) (layer B.Cu) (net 19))
 (segment (start 74.295 89.9795) (end 74.295 86.995) (width 0.25) (layer B.Cu) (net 19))
 (segment (start 75.565 91.2495) (end 74.295 89.9795) (width 0.25) (layer B.Cu) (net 19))
 (via (at 75.565 91.2495) (size 0.6) (drill 0.4) (layers F.Cu B.Cu) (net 19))
 (segment (start 75.5345 91.28) (end 75.565 91.2495) (width 0.25) (layer F.Cu) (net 19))
 (segment (start 75.78 89.18) (end 74.702 89.18) (width 0.25) (layer F.Cu) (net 20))
 (segment (start 73.406 87.884) (end 73.406 83.566) (width 0.25) (layer F.Cu) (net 20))
 (segment (start 74.702 89.18) (end 73.406 87.884) (width 0.25) (layer F.Cu) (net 20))
 (segment (start 73.406 83.566) (end 71.12 81.28) (width 0.25) (layer F.Cu) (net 20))
 (segment (start 77.98 89.18) (end 77.98 86.743) (width 0.25) (layer F.Cu) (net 21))
 (segment (start 73.025 80.645) (end 71.12 78.74) (width 0.25) (layer F.Cu) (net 21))
 (segment (start 73.025 81.788) (end 73.025 80.645) (width 0.25) (layer F.Cu) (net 21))
 (segment (start 77.98 86.743) (end 73.025 81.788) (width 0.25) (layer F.Cu) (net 21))
 (segment (start 79.08 89.18) (end 79.08 86.446) (width 0.25) (layer F.Cu) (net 22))
 (segment (start 73.8505 81.2165) (end 73.8505 78.9305) (width 0.25) (layer F.Cu) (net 22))
 (segment (start 79.08 86.446) (end 73.8505 81.2165) (width 0.25) (layer F.Cu) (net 22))
 (segment (start 73.8505 78.9305) (end 71.12 76.2) (width 0.25) (layer F.Cu) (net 22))
 (segment (start 71.12 73.66) (end 72.39 73.66) (width 0.25) (layer F.Cu) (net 23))
 (segment (start 73.152 76.962) (end 74.7395 78.5495) (width 0.25) (layer F.Cu) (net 23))
 (segment (start 73.152 74.422) (end 73.152 76.962) (width 0.25) (layer F.Cu) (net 23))
 (segment (start 72.39 73.66) (end 73.152 74.422) (width 0.25) (layer F.Cu) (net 23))
 (segment (start 80.18 89.18) (end 80.18 85.9585) (width 0.25) (layer F.Cu) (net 23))
 (segment (start 74.7395 80.518) (end 74.7395 78.5495) (width 0.25) (layer F.Cu) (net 23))
 (segment (start 80.18 85.9585) (end 74.7395 80.518) (width 0.25) (layer F.Cu) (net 23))
 (segment (start 71.12 71.12) (end 74.168 74.168) (width 0.25) (layer F.Cu) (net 24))
 (segment (start 75.7555 78.232) (end 75.7555 77.7875) (width 0.25) (layer F.Cu) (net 24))
 (segment (start 75.7555 77.7875) (end 74.168 76.2) (width 0.25) (layer F.Cu) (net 24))
 (segment (start 74.168 76.2) (end 74.168 74.168) (width 0.25) (layer F.Cu) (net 24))
 (segment (start 81.28 85.725) (end 81.28 89.18) (width 0.25) (layer F.Cu) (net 24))
 (segment (start 75.7555 80.2005) (end 81.28 85.725) (width 0.25) (layer F.Cu) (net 24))
 (segment (start 75.7555 78.232) (end 75.7555 80.2005) (width 0.25) (layer F.Cu) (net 24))
 (segment (start 82.38 89.18) (end 82.38 86.784) (width 0.25) (layer F.Cu) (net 25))
 (segment (start 88.9 80.264) (end 88.9 76.2) (width 0.25) (layer F.Cu) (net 25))
 (segment (start 82.38 86.784) (end 88.9 80.264) (width 0.25) (layer F.Cu) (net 25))
 (segment (start 88.9 76.2) (end 93.98 71.12) (width 0.25) (layer F.Cu) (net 25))
 (segment (start 83.48 89.18) (end 83.48 87.335) (width 0.25) (layer F.Cu) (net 26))
 (segment (start 90.043 80.772) (end 90.043 77.597) (width 0.25) (layer F.Cu) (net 26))
 (segment (start 83.48 87.335) (end 90.043 80.772) (width 0.25) (layer F.Cu) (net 26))
 (segment (start 90.043 77.597) (end 93.98 73.66) (width 0.25) (layer F.Cu) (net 26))
 (segment (start 84.58 89.18) (end 84.58 87.886) (width 0.25) (layer F.Cu) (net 27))
 (segment (start 91.059 81.407) (end 91.059 79.121) (width 0.25) (layer F.Cu) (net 27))
 (segment (start 84.58 87.886) (end 91.059 81.407) (width 0.25) (layer F.Cu) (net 27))
 (segment (start 91.059 79.121) (end 93.98 76.2) (width 0.25) (layer F.Cu) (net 27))
 (segment (start 85.68 89.18) (end 85.68 87.8655) (width 0.25) (layer F.Cu) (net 28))
 (segment (start 91.821 80.899) (end 93.98 78.74) (width 0.25) (layer F.Cu) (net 28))
 (segment (start 91.821 81.7245) (end 91.821 80.899) (width 0.25) (layer F.Cu) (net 28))
 (segment (start 85.68 87.8655) (end 91.821 81.7245) (width 0.25) (layer F.Cu) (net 28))
 (segment (start 93.98 78.74) (end 93.7895 78.74) (width 0.25) (layer F.Cu) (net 28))
 (segment (start 87.88 89.18) (end 87.88 87.38) (width 0.25) (layer F.Cu) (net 29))
 (segment (start 87.88 87.38) (end 93.98 81.28) (width 0.25) (layer F.Cu) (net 29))
 (segment (start 90.66 92.38) (end 88.595 92.38) (width 0.25) (layer F.Cu) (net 30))
 (segment (start 90.9955 86.8045) (end 93.98 83.82) (width 0.25) (layer B.Cu) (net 30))
 (segment (start 90.9955 91.44) (end 90.9955 86.8045) (width 0.25) (layer B.Cu) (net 30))
 (segment (start 90.043 92.3925) (end 90.9955 91.44) (width 0.25) (layer B.Cu) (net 30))
 (segment (start 88.5825 92.3925) (end 90.043 92.3925) (width 0.25) (layer B.Cu) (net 30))
 (segment (start 88.519 92.456) (end 88.5825 92.3925) (width 0.25) (layer B.Cu) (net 30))
 (via (at 88.519 92.456) (size 0.6) (drill 0.4) (layers F.Cu B.Cu) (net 30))
 (segment (start 88.595 92.38) (end 88.519 92.456) (width 0.25) (layer F.Cu) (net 30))
 (segment (start 93.98 86.36) (end 93.726 86.36) (width 0.25) (layer B.Cu) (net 31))
 (segment (start 93.726 86.36) (end 91.948 88.138) (width 0.25) (layer B.Cu) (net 31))
 (segment (start 91.948 88.138) (end 91.948 91.694) (width 0.25) (layer B.Cu) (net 31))
 (segment (start 91.948 91.694) (end 90.17 93.472) (width 0.25) (layer B.Cu) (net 31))
 (segment (start 90.17 93.472) (end 88.5825 93.472) (width 0.25) (layer B.Cu) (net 31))
 (via (at 88.5825 93.472) (size 0.6) (drill 0.4) (layers F.Cu B.Cu) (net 31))
 (segment (start 88.5825 93.472) (end 88.5905 93.48) (width 0.25) (layer F.Cu) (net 31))
 (segment (start 88.5905 93.48) (end 90.66 93.48) (width 0.25) (layer F.Cu) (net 31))
 (segment (start 90.66 96.78) (end 92.0055 96.78) (width 0.25) (layer F.Cu) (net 34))
 (segment (start 92.202 95.758) (end 93.98 93.98) (width 0.25) (layer F.Cu) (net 34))
 (segment (start 92.202 96.5835) (end 92.202 95.758) (width 0.25) (layer F.Cu) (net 34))
 (segment (start 92.0055 96.78) (end 92.202 96.5835) (width 0.25) (layer F.Cu) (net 34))
 (segment (start 90.66 97.88) (end 92.62 97.88) (width 0.25) (layer F.Cu) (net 35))
 (segment (start 92.62 97.88) (end 93.98 96.52) (width 0.25) (layer F.Cu) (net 35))
 (segment (start 90.66 98.98) (end 93.9 98.98) (width 0.25) (layer F.Cu) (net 36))
 (segment (start 93.9 98.98) (end 93.98 99.06) (width 0.25) (layer F.Cu) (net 36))
 (segment (start 90.66 100.08) (end 92.46 100.08) (width 0.25) (layer F.Cu) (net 37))
 (segment (start 92.46 100.08) (end 93.98 101.6) (width 0.25) (layer F.Cu) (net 37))
 (segment (start 93.98 104.14) (end 93.98 104.0765) (width 0.25) (layer B.Cu) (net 38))
 (segment (start 93.98 104.0765) (end 91.059 101.1555) (width 0.25) (layer B.Cu) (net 38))
 (segment (start 91.059 101.1555) (end 88.7095 101.1555) (width 0.25) (layer B.Cu) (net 38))
 (via (at 88.7095 101.1555) (size 0.6) (drill 0.4) (layers F.Cu B.Cu) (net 38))
 (segment (start 88.7095 101.1555) (end 88.734 101.18) (width 0.25) (layer F.Cu) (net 38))
 (segment (start 88.734 101.18) (end 90.66 101.18) (width 0.25) (layer F.Cu) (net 38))
 (segment (start 90.66 102.28) (end 88.818 102.28) (width 0.25) (layer F.Cu) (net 39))
 (segment (start 92.1385 104.8385) (end 93.98 106.68) (width 0.25) (layer B.Cu) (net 39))
 (segment (start 92.1385 103.378) (end 92.1385 104.8385) (width 0.25) (layer B.Cu) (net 39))
 (segment (start 90.9955 102.235) (end 92.1385 103.378) (width 0.25) (layer B.Cu) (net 39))
 (segment (start 88.773 102.235) (end 90.9955 102.235) (width 0.25) (layer B.Cu) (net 39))
 (segment (start 88.7095 102.1715) (end 88.773 102.235) (width 0.25) (layer B.Cu) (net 39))
 (via (at 88.7095 102.1715) (size 0.6) (drill 0.4) (layers F.Cu B.Cu) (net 39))
 (segment (start 88.818 102.28) (end 88.7095 102.1715) (width 0.25) (layer F.Cu) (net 39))
 (segment (start 93.98 109.22) (end 93.599 109.22) (width 0.25) (layer B.Cu) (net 40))
 (segment (start 93.599 109.22) (end 91.3765 106.9975) (width 0.25) (layer B.Cu) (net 40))
 (segment (start 91.3765 106.9975) (end 91.3765 103.886) (width 0.25) (layer B.Cu) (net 40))
 (segment (start 91.3765 103.886) (end 90.8685 103.378) (width 0.25) (layer B.Cu) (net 40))
 (segment (start 90.8685 103.378) (end 88.773 103.378) (width 0.25) (layer B.Cu) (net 40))
 (via (at 88.773 103.378) (size 0.6) (drill 0.4) (layers F.Cu B.Cu) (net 40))
 (segment (start 88.773 103.378) (end 88.775 103.38) (width 0.25) (layer F.Cu) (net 40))
 (segment (start 88.775 103.38) (end 90.66 103.38) (width 0.25) (layer F.Cu) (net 40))
 (segment (start 90.66 104.48) (end 90.66 104.5665) (width 0.25) (layer F.Cu) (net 41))
 (segment (start 90.66 104.5665) (end 91.7575 105.664) (width 0.25) (layer F.Cu) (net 41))
 (segment (start 91.7575 105.664) (end 91.7575 109.5375) (width 0.25) (layer F.Cu) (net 41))
 (segment (start 91.7575 109.5375) (end 93.98 111.76) (width 0.25) (layer F.Cu) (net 41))
 (segment (start 89.98 106.68) (end 89.98 110.3) (width 0.25) (layer F.Cu) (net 42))
 (segment (start 89.98 110.3) (end 93.98 114.3) (width 0.25) (layer F.Cu) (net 42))
 (segment (start 88.98 106.68) (end 88.98 111.84) (width 0.25) (layer F.Cu) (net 43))
 (segment (start 88.98 111.84) (end 93.98 116.84) (width 0.25) (layer F.Cu) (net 43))
 (segment (start 87.98 106.68) (end 87.98 113.38) (width 0.25) (layer F.Cu) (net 44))
 (segment (start 87.98 113.38) (end 93.98 119.38) (width 0.25) (layer F.Cu) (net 44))
 (segment (start 86.93 106.68) (end 86.93 114.87) (width 0.25) (layer F.Cu) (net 45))
 (segment (start 86.93 114.87) (end 93.98 121.92) (width 0.25) (layer F.Cu) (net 45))
 (segment (start 85.83 106.68) (end 85.83 116.31) (width 0.25) (layer F.Cu) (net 46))
 (segment (start 85.83 116.31) (end 93.98 124.46) (width 0.25) (layer F.Cu) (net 46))
 (segment (start 82.53 106.68) (end 82.53 115.55) (width 0.25) (layer F.Cu) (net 47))
 (segment (start 82.53 115.55) (end 93.98 127) (width 0.25) (layer F.Cu) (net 47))
 (segment (start 90.66 91.28) (end 88.2472 91.28) (width 0.25) (layer F.Cu) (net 14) (status 400000))
 (segment (start 80.1878 73.2282) (end 82.042 71.374) (width 0.25) (layer B.Cu) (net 14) (status 800000))
 (segment (start 76.1746 73.2282) (end 80.1878 73.2282) (width 0.25) (layer B.Cu) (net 14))
 (segment (start 74.3712 75.0316) (end 76.1746 73.2282) (width 0.25) (layer B.Cu) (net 14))
 (segment (start 74.3712 84.7344) (end 74.3712 75.0316) (width 0.25) (layer B.Cu) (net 14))
 (segment (start 76.4794 86.8426) (end 74.3712 84.7344) (width 0.25) (layer B.Cu) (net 14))
 (segment (start 76.4794 90.678) (end 76.4794 86.8426) (width 0.25) (layer B.Cu) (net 14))
 (segment (start 78.5368 92.7354) (end 76.4794 90.678) (width 0.25) (layer B.Cu) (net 14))
 (via (at 78.5368 92.7354) (size 0.6) (drill 0.4) (layers F.Cu B.Cu) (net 14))
 (segment (start 79.2734 93.472) (end 78.5368 92.7354) (width 0.25) (layer F.Cu) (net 14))
 (segment (start 86.0552 93.472) (end 79.2734 93.472) (width 0.25) (layer F.Cu) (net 14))
 (segment (start 88.2472 91.28) (end 86.0552 93.472) (width 0.25) (layer F.Cu) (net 14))
 (segment (start 83.63 106.68) (end 84.73 106.68) (width 0.25) (layer F.Cu) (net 14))
 (segment (start 84.73 106.68) (end 84.73 103.7165) (width 0.25) (layer F.Cu) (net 14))
 (segment (start 84.6875 103.759) (end 76.9925 103.759) (width 0.25) (layer F.Cu) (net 14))
 (segment (start 84.73 103.7165) (end 84.6875 103.759) (width 0.25) (layer F.Cu) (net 14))
 (segment (start 76.9925 96.7435) (end 76.9925 103.759) (width 0.25) (layer F.Cu) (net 14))
 (segment (start 76.9925 103.759) (end 76.9925 103.792) (width 0.25) (layer F.Cu) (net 14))
 (segment (start 75.93 104.8545) (end 75.93 106.68) (width 0.25) (layer F.Cu) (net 14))
 (segment (start 76.9925 103.792) (end 75.93 104.8545) (width 0.25) (layer F.Cu) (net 14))
 (segment (start 73.66 96.78) (end 71.38 96.78) (width 0.25) (layer F.Cu) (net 14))
 (segment (start 71.38 96.78) (end 71.12 96.52) (width 0.25) (layer F.Cu) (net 14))
 (segment (start 76.9925 91.28) (end 76.9925 96.7435) (width 0.25) (layer F.Cu) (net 14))
 (segment (start 76.956 96.78) (end 73.66 96.78) (width 0.25) (layer F.Cu) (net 14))
 (segment (start 76.9925 96.7435) (end 76.956 96.78) (width 0.25) (layer F.Cu) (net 14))
 (segment (start 86.741 91.28) (end 76.9925 91.28) (width 0.25) (layer F.Cu) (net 14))
 (segment (start 76.88 91.1675) (end 76.88 89.18) (width 0.25) (layer F.Cu) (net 14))
 (segment (start 76.9925 91.28) (end 76.88 91.1675) (width 0.25) (layer F.Cu) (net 14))
 (segment (start 86.741 91.28) (end 86.708 91.28) (width 0.25) (layer F.Cu) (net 14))
 (segment (start 86.78 91.208) (end 86.78 89.18) (width 0.25) (layer F.Cu) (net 14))
 (segment (start 86.708 91.28) (end 86.78 91.208) (width 0.25) (layer F.Cu) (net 14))
 (segment (start 93.98 88.9) (end 90.678 88.9) (width 0.25) (layer F.Cu) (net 32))
 (segment (start 87.042 85.264) (end 87.042 76.374) (width 0.25) (layer B.Cu) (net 32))
 (segment (start 89.662 87.884) (end 87.042 85.264) (width 0.25) (layer B.Cu) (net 32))
 (via (at 89.662 87.884) (size 0.6) (drill 0.4) (layers F.Cu B.Cu) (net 32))
 (segment (start 90.678 88.9) (end 89.662 87.884) (width 0.25) (layer F.Cu) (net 32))
 (segment (start 90.66 94.58) (end 92.0465 94.58) (width 0.25) (layer F.Cu) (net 32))
 (segment (start 92.202 90.678) (end 93.98 88.9) (width 0.25) (layer F.Cu) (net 32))
 (segment (start 92.202 94.4245) (end 92.202 90.678) (width 0.25) (layer F.Cu) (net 32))
 (segment (start 92.0465 94.58) (end 92.202 94.4245) (width 0.25) (layer F.Cu) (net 32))
 (segment (start 77.042 76.374) (end 77.042 84.2175) (width 0.25) (layer B.Cu) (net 33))
 (segment (start 77.042 84.2175) (end 88.519 95.6945) (width 0.25) (layer B.Cu) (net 33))
 (segment (start 90.66 95.68) (end 88.5335 95.68) (width 0.25) (layer F.Cu) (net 33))
 (segment (start 91.948 93.472) (end 93.98 91.44) (width 0.25) (layer B.Cu) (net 33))
 (segment (start 91.948 94.869) (end 91.948 93.472) (width 0.25) (layer B.Cu) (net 33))
 (segment (start 91.1225 95.6945) (end 91.948 94.869) (width 0.25) (layer B.Cu) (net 33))
 (segment (start 88.519 95.6945) (end 91.1225 95.6945) (width 0.25) (layer B.Cu) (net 33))
 (via (at 88.519 95.6945) (size 0.6) (drill 0.4) (layers F.Cu B.Cu) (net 33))
 (segment (start 88.5335 95.68) (end 88.519 95.6945) (width 0.25) (layer F.Cu) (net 33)))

